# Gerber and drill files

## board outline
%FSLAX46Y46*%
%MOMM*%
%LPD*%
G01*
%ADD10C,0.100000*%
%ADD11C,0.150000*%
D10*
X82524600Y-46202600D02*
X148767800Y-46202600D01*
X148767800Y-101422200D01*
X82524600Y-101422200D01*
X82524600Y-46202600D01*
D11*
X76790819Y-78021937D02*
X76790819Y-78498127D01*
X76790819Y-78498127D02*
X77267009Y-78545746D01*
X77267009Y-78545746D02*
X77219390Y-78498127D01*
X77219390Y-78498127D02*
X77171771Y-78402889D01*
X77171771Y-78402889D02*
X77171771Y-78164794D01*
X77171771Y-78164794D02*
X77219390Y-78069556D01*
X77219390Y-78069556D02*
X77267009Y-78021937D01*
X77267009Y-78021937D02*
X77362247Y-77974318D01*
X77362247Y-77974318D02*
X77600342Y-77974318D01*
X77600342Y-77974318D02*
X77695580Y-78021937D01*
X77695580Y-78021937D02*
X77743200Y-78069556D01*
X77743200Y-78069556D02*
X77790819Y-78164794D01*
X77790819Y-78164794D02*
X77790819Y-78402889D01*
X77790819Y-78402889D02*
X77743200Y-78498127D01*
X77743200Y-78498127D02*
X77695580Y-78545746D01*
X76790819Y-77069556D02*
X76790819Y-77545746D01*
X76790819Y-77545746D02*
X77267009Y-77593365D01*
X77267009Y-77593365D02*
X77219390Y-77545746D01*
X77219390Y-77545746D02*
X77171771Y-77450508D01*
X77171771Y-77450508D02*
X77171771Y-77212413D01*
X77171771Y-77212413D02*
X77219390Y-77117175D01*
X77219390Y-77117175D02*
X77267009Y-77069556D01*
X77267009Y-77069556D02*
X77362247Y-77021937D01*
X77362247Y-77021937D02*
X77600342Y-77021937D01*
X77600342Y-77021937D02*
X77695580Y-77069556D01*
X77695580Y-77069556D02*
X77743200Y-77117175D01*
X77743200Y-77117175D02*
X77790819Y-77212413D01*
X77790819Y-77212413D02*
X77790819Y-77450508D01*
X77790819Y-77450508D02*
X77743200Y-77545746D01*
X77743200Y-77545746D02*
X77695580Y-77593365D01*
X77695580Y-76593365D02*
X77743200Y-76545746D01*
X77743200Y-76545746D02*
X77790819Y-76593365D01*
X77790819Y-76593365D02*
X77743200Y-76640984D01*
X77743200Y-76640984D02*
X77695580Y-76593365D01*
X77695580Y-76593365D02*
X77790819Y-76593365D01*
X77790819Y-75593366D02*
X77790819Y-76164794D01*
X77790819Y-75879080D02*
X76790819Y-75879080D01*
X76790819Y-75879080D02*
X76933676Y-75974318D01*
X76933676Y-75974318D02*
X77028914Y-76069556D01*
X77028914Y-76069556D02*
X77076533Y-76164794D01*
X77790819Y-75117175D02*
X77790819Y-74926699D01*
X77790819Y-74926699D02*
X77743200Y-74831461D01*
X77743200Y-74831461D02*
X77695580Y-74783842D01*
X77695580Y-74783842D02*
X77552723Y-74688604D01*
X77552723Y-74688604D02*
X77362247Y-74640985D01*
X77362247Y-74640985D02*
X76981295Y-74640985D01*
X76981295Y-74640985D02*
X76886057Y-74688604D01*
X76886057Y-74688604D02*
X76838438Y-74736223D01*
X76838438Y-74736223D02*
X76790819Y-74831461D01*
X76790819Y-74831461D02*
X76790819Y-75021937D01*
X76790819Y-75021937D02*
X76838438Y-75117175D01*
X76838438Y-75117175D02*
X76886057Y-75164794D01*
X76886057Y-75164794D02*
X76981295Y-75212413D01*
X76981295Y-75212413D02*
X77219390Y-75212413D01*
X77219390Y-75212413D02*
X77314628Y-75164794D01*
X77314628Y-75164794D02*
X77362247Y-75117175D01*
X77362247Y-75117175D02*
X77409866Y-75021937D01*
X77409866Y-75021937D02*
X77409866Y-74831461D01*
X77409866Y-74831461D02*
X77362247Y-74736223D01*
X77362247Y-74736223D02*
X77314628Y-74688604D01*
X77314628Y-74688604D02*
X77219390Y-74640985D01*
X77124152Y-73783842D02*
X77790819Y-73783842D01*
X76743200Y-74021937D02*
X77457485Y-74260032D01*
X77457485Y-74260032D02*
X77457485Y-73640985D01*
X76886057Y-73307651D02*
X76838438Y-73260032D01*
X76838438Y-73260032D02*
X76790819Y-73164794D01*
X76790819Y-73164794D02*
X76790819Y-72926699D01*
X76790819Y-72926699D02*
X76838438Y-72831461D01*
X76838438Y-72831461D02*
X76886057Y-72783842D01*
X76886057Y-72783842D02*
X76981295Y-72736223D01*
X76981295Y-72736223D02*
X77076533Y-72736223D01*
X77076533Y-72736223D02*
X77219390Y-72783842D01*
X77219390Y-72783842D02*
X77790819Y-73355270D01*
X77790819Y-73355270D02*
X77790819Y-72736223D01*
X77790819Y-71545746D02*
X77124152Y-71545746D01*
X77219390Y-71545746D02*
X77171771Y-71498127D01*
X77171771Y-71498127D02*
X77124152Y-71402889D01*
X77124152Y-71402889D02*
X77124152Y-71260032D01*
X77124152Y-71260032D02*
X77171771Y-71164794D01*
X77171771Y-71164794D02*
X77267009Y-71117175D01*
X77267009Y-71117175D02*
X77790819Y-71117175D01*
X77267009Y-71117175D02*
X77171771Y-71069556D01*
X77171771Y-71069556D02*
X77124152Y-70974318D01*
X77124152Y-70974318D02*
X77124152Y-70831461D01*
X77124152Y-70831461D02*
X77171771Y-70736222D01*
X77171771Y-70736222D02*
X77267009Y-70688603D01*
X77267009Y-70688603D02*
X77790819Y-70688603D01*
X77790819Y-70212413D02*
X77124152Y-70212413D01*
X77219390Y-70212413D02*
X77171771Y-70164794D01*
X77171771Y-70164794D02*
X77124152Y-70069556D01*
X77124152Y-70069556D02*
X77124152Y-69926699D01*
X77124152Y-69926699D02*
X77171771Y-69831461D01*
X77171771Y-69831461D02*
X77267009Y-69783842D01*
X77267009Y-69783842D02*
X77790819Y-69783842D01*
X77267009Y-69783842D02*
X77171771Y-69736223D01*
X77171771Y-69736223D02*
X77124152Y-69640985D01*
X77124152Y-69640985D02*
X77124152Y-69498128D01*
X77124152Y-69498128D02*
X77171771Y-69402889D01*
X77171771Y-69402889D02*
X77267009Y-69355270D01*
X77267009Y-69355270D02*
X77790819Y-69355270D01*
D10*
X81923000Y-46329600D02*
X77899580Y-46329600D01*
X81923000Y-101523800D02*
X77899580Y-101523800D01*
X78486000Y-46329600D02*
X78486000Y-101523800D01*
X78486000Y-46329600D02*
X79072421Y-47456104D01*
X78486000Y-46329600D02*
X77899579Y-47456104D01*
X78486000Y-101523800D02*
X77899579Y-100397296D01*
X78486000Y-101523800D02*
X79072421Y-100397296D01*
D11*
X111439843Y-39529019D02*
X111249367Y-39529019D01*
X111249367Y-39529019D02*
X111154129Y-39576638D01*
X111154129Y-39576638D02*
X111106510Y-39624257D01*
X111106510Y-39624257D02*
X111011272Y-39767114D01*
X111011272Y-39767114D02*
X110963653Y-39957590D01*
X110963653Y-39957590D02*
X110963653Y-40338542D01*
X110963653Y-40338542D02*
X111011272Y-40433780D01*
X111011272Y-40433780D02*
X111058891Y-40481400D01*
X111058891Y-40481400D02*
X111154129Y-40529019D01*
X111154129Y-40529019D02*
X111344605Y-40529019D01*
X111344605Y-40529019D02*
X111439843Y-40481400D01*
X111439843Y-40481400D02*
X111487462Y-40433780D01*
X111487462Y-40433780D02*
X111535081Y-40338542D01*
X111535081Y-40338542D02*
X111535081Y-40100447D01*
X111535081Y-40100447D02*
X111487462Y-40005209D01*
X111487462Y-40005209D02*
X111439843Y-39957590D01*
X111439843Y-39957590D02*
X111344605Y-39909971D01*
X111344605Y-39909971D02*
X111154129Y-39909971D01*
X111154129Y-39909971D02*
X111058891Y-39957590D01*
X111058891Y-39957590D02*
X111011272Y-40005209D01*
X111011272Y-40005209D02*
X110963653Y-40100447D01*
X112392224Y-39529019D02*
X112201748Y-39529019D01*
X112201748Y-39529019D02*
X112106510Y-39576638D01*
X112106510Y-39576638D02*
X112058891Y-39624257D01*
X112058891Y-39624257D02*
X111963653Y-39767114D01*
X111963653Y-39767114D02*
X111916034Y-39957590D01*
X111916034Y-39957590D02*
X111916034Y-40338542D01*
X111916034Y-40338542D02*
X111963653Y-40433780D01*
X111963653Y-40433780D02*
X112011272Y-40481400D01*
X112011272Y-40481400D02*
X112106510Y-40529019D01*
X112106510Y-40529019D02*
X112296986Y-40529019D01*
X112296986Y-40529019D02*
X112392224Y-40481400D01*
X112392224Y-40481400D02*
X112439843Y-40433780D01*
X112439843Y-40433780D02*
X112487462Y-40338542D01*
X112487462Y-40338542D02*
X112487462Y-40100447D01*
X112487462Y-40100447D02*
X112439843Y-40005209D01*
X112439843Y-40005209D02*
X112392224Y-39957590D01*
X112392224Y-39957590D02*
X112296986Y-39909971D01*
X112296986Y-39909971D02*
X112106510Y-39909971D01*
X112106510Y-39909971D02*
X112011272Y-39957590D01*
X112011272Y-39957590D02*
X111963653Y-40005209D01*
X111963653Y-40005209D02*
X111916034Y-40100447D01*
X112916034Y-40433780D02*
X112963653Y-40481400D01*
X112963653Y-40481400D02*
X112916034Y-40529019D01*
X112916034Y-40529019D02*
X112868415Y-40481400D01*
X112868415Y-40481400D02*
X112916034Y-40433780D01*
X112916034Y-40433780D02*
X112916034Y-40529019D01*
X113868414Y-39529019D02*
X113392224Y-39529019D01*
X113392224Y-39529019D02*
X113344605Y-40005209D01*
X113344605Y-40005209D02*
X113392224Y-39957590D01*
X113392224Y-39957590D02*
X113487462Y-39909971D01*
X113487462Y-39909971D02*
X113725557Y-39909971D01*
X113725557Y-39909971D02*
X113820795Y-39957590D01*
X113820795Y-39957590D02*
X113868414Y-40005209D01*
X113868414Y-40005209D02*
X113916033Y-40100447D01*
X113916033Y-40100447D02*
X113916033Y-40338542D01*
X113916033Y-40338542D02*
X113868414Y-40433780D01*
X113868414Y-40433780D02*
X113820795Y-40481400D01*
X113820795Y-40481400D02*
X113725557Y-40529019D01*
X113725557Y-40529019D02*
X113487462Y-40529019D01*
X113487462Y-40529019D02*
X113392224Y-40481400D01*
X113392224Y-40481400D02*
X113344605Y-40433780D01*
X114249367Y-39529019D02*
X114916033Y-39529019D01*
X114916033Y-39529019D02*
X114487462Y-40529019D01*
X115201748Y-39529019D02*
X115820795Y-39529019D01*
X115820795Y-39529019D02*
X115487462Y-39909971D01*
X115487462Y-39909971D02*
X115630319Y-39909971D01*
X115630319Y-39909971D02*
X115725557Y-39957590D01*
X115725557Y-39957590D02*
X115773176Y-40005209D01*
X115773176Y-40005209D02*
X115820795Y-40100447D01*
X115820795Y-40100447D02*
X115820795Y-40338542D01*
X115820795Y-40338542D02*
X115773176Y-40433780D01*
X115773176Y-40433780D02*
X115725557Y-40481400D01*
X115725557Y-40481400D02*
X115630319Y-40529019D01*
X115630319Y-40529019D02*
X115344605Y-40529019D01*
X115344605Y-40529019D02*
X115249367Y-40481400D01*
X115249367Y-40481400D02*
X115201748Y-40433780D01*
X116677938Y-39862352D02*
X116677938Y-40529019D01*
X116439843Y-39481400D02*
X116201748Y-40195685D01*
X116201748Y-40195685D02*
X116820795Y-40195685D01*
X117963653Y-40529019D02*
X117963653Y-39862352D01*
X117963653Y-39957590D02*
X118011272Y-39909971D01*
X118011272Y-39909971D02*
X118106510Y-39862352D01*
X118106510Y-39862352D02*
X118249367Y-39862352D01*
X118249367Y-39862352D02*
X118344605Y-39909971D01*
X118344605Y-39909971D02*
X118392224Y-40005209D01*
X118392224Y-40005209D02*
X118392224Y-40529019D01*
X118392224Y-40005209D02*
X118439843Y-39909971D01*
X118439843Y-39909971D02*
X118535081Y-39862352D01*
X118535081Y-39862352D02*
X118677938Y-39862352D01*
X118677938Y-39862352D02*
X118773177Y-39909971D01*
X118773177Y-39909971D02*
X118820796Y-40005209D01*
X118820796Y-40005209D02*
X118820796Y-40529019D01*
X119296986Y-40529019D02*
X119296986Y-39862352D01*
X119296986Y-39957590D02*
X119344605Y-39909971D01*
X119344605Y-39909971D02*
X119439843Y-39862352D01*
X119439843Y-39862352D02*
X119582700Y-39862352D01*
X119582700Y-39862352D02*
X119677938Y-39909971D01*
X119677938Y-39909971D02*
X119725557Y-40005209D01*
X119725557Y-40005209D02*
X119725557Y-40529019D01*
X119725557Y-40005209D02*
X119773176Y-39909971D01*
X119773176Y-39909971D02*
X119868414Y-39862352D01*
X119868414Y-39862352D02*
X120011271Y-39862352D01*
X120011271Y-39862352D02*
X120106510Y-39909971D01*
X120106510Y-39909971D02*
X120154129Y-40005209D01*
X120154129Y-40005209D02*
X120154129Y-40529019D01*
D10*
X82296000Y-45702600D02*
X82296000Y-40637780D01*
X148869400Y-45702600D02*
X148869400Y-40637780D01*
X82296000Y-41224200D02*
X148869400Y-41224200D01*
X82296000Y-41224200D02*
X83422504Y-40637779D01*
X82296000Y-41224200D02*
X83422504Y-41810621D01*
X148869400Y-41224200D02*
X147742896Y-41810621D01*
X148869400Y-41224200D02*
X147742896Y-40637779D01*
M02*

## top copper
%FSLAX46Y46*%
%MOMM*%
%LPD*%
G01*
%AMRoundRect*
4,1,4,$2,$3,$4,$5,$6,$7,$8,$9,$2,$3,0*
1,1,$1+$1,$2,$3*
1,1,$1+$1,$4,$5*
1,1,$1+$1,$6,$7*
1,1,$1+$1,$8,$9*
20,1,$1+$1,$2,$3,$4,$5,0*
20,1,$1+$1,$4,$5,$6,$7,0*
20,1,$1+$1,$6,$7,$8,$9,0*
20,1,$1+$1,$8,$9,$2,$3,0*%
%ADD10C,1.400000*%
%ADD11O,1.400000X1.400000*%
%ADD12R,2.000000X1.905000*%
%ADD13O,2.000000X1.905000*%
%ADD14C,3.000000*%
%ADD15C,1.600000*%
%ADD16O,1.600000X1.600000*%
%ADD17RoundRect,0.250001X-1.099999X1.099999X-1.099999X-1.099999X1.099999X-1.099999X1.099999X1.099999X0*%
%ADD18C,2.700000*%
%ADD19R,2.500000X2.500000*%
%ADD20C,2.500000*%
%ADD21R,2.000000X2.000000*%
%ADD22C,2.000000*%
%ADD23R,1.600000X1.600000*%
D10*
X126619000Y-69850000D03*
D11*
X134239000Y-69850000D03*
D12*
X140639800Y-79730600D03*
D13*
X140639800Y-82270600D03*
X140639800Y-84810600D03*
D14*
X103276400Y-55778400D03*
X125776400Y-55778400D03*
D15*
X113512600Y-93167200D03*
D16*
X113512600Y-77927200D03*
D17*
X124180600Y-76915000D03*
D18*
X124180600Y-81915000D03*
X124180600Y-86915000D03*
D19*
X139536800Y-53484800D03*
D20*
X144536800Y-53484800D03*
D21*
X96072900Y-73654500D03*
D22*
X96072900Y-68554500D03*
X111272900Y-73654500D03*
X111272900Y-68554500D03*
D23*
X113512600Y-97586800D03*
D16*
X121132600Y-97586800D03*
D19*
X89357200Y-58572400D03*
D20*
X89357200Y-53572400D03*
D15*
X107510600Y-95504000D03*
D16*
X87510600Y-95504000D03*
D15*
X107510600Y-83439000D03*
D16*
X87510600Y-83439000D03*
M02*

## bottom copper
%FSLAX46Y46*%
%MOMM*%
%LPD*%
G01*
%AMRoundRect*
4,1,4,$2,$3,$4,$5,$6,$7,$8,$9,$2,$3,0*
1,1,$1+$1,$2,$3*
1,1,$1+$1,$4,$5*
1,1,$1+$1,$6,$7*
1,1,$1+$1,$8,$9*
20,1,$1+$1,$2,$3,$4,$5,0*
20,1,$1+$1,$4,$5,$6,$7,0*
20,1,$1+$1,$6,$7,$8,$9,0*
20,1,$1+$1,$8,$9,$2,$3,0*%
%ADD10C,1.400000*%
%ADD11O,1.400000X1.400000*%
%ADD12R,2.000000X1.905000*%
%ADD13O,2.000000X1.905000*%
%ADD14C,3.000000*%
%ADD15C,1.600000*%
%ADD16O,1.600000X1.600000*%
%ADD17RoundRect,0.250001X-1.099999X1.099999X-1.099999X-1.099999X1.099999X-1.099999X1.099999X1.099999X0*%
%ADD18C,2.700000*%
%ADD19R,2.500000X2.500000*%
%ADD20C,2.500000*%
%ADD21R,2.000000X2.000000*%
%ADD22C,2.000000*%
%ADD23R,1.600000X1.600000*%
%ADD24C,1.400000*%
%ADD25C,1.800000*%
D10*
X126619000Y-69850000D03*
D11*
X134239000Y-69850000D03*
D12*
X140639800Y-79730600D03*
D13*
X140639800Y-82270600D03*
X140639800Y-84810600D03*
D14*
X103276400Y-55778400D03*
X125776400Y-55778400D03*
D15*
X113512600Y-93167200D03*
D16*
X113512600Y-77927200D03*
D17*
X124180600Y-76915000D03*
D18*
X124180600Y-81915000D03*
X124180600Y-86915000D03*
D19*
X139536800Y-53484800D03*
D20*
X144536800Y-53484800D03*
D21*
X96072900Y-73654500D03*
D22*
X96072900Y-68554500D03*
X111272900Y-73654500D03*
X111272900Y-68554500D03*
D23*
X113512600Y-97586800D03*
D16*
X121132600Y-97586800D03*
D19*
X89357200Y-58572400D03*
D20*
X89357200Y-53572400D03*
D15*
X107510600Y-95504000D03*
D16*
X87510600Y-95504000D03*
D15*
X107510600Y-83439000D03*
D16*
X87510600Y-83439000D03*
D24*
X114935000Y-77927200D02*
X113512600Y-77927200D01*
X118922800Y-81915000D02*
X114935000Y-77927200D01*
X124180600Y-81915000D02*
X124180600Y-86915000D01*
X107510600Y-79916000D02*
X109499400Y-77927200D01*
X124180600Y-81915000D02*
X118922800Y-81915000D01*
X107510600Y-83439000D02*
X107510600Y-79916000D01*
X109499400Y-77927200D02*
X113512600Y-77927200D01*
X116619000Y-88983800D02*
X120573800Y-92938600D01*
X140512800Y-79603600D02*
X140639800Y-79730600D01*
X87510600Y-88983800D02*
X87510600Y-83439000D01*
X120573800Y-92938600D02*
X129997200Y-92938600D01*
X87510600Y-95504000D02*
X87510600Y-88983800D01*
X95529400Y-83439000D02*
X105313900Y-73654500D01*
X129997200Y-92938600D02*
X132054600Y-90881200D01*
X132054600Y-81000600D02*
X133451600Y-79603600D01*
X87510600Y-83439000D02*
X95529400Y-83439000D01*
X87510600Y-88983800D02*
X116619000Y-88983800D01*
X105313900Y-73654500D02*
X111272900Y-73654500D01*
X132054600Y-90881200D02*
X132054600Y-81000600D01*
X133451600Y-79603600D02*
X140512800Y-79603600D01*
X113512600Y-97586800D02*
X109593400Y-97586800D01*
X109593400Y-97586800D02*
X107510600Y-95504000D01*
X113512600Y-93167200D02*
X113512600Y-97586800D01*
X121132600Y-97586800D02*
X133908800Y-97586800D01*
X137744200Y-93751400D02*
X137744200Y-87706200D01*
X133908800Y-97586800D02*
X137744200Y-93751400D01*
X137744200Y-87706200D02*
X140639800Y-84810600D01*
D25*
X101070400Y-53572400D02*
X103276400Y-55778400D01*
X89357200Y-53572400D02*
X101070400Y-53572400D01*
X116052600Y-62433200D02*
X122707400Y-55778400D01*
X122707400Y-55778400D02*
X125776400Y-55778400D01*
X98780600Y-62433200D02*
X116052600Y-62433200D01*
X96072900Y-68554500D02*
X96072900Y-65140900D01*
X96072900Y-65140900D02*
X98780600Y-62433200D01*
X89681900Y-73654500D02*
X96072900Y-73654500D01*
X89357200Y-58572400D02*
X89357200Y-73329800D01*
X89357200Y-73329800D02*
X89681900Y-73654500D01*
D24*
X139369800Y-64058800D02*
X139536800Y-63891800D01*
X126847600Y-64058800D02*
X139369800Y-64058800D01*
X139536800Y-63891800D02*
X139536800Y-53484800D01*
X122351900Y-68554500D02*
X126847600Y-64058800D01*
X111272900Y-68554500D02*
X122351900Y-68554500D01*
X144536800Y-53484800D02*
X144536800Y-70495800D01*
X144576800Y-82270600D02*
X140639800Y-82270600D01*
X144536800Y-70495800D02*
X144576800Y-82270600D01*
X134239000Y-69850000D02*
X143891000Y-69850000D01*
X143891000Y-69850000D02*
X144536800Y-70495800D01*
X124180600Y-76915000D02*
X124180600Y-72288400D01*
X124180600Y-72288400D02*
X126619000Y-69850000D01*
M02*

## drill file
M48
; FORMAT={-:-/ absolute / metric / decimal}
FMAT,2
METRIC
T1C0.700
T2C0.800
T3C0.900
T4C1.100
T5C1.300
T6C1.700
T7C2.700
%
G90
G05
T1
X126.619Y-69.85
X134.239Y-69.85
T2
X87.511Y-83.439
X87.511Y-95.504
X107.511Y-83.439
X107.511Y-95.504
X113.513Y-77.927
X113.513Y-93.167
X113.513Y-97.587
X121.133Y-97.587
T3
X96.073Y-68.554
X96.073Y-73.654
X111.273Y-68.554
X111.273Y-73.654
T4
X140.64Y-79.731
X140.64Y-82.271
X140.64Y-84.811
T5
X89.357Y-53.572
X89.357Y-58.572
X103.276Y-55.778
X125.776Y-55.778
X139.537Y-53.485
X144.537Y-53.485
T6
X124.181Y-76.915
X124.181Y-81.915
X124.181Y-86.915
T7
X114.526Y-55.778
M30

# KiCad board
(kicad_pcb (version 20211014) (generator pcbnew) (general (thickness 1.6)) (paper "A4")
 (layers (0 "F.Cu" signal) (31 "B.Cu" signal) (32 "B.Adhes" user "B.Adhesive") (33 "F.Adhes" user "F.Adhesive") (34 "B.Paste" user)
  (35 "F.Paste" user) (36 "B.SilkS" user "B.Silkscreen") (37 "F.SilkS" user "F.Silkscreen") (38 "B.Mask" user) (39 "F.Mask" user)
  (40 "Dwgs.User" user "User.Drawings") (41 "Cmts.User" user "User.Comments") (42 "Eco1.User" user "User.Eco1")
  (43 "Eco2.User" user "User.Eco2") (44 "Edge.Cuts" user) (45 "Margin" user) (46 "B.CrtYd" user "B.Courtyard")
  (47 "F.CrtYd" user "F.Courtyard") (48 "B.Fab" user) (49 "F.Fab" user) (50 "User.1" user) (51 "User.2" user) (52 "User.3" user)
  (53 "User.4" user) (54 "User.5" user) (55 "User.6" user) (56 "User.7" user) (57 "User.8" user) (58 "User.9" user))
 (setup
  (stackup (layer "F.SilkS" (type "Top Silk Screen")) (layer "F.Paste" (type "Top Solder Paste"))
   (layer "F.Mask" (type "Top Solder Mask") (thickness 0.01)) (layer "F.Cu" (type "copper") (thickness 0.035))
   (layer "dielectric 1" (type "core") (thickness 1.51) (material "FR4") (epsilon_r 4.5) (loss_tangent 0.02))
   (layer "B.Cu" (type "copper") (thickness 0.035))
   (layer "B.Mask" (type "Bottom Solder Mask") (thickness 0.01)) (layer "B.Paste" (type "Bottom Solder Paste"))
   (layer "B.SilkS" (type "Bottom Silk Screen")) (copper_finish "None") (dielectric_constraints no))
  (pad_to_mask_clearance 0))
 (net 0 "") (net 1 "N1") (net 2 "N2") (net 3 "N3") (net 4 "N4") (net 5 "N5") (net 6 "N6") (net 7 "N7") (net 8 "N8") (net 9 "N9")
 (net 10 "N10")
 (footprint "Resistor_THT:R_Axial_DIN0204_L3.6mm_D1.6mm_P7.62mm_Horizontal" (layer "F.Cu") (at 126.619 69.85)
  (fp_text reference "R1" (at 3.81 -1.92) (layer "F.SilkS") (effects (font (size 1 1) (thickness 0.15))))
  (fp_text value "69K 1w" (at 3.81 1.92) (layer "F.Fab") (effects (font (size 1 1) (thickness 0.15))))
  (pad "1" thru_hole circle (at 0 0) (size 1.4 1.4) (drill 0.7) (layers *.Cu *.Mask) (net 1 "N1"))
  (pad "2" thru_hole oval (at 7.62 0) (size 1.4 1.4) (drill 0.7) (layers *.Cu *.Mask) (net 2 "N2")))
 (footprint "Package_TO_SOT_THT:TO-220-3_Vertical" (layer "F.Cu") (at 140.6398 79.7306 -90)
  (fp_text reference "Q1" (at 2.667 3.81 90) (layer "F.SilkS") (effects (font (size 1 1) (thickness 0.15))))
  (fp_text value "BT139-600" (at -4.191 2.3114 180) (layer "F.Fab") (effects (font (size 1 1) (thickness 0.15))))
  (pad "1" thru_hole rect (at 0 0 270) (size 1.905 2) (drill 1.1) (layers *.Cu *.Mask) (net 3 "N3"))
  (pad "2" thru_hole oval (at 2.54 0 270) (size 1.905 2) (drill 1.1) (layers *.Cu *.Mask) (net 2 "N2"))
  (pad "3" thru_hole oval (at 5.08 0 270) (size 1.905 2) (drill 1.1) (layers *.Cu *.Mask) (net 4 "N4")))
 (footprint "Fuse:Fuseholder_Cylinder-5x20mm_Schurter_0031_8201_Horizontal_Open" (layer "F.Cu") (at 103.2764 55.7784)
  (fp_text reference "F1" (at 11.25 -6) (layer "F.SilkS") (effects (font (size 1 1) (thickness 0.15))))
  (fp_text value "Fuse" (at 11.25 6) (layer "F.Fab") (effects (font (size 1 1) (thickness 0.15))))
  (pad "" np_thru_hole circle (at 11.25 0) (size 2.7 2.7) (drill 2.7) (layers *.Cu *.Mask))
  (pad "1" thru_hole circle (at 0 0) (size 3 3) (drill 1.3) (layers *.Cu *.Mask) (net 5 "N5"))
  (pad "2" thru_hole circle (at 22.5 0) (size 3 3) (drill 1.3) (layers *.Cu *.Mask) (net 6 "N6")))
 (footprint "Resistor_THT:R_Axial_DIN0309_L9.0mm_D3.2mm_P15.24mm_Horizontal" (layer "F.Cu") (at 113.5126 93.1672 90)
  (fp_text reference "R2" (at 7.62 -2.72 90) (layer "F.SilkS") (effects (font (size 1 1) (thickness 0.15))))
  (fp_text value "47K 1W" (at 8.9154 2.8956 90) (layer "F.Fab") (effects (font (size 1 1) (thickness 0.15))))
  (pad "1" thru_hole circle (at 0 0 90) (size 1.6 1.6) (drill 0.8) (layers *.Cu *.Mask) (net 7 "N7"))
  (pad "2" thru_hole oval (at 15.24 0 90) (size 1.6 1.6) (drill 0.8) (layers *.Cu *.Mask) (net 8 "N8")))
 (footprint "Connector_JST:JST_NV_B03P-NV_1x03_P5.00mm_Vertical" (layer "F.Cu") (at 124.1806 76.915 -90)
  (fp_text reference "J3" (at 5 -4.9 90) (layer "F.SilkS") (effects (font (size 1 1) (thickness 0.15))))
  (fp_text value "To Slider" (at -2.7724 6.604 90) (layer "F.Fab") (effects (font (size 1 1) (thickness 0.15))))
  (pad "1" thru_hole roundrect (at 0 0 270) (size 2.7 2.7) (drill 1.7) (layers *.Cu *.Mask) (roundrect_rratio 0.092593) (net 1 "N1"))
  (pad "2" thru_hole circle (at 5 0 270) (size 2.7 2.7) (drill 1.7) (layers *.Cu *.Mask) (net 8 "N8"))
  (pad "3" thru_hole circle (at 10 0 270) (size 2.7 2.7) (drill 1.7) (layers *.Cu *.Mask) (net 8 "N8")))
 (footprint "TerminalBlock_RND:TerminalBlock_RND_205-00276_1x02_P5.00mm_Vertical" (layer "F.Cu") (at 139.5368 53.4848)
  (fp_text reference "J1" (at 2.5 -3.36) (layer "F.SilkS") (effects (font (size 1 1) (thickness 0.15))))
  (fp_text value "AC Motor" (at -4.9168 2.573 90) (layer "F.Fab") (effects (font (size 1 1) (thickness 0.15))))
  (pad "1" thru_hole rect (at 0 0) (size 2.5 2.5) (drill 1.3) (layers *.Cu *.Mask) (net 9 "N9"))
  (pad "2" thru_hole circle (at 5 0) (size 2.5 2.5) (drill 1.3) (layers *.Cu *.Mask) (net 2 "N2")))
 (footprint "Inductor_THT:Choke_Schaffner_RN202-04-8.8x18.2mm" (layer "F.Cu") (at 96.0729 73.6545 90)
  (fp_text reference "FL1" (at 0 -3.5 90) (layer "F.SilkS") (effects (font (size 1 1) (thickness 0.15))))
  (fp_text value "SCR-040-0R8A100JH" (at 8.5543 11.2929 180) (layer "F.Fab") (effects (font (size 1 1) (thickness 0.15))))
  (pad "1" thru_hole rect (at 0 0 90) (size 2 2) (drill 0.9) (layers *.Cu *.Mask) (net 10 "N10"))
  (pad "2" thru_hole circle (at 5.1 0 90) (size 2 2) (drill 0.9) (layers *.Cu *.Mask) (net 6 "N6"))
  (pad "3" thru_hole circle (at 0 15.2 90) (size 2 2) (drill 0.9) (layers *.Cu *.Mask) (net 3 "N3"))
  (pad "4" thru_hole circle (at 5.1 15.2 90) (size 2 2) (drill 0.9) (layers *.Cu *.Mask) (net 9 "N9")))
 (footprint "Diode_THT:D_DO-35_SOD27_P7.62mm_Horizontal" (layer "F.Cu") (at 113.5126 97.5868)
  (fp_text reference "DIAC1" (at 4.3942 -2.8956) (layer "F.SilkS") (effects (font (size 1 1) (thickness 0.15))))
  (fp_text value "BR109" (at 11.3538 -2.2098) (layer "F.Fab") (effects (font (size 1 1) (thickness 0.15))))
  (pad "1" thru_hole rect (at 0 0) (size 1.6 1.6) (drill 0.8) (layers *.Cu *.Mask) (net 7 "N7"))
  (pad "2" thru_hole oval (at 7.62 0) (size 1.6 1.6) (drill 0.8) (layers *.Cu *.Mask) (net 4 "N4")))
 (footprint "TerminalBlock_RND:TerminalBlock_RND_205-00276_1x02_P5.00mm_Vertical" (layer "F.Cu") (at 89.3572 58.5724 90)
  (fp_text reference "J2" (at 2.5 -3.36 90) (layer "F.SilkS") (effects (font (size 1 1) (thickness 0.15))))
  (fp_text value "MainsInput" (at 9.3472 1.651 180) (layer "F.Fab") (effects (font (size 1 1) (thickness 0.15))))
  (pad "1" thru_hole rect (at 0 0 90) (size 2.5 2.5) (drill 1.3) (layers *.Cu *.Mask) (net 10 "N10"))
  (pad "2" thru_hole circle (at 5 0 90) (size 2.5 2.5) (drill 1.3) (layers *.Cu *.Mask) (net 5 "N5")))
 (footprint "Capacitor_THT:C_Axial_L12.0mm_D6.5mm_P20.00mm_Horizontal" (layer "F.Cu") (at 107.5106 95.504 180)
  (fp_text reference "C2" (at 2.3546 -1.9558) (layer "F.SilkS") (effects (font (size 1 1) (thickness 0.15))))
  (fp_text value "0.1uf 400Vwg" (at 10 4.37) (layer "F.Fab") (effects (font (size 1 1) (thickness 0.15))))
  (pad "1" thru_hole circle (at 0 0 180) (size 1.6 1.6) (drill 0.8) (layers *.Cu *.Mask) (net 7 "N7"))
  (pad "2" thru_hole oval (at 20 0 180) (size 1.6 1.6) (drill 0.8) (layers *.Cu *.Mask) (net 3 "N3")))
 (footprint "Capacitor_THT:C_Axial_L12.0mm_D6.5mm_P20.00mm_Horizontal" (layer "F.Cu") (at 107.5106 83.439 180)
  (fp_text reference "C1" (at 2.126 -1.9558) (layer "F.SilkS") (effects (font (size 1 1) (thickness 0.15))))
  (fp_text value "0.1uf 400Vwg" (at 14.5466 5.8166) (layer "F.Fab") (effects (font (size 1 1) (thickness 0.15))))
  (pad "1" thru_hole circle (at 0 0 180) (size 1.6 1.6) (drill 0.8) (layers *.Cu *.Mask) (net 8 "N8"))
  (pad "2" thru_hole oval (at 20 0 180) (size 1.6 1.6) (drill 0.8) (layers *.Cu *.Mask) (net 3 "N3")))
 (gr_rect (start 82.5246 46.2026) (end 148.7678 101.4222) (layer "Edge.Cuts") (width 0.1) (fill none))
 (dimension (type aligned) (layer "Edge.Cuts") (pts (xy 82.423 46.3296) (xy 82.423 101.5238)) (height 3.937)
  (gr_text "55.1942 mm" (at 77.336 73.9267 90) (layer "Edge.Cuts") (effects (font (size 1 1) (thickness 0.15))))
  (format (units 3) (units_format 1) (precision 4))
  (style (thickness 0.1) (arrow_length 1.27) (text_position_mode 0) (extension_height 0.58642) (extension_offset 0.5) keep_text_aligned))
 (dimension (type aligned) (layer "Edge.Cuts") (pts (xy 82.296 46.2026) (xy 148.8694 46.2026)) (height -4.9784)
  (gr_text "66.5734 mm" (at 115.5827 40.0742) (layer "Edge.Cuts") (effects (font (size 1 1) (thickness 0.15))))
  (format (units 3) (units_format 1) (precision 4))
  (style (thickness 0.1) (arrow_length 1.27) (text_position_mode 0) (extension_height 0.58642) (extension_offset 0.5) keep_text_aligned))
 (segment (start 114.935 77.9272) (end 113.5126 77.9272) (width 1.4) (layer "B.Cu") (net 8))
 (segment (start 118.9228 81.915) (end 114.935 77.9272) (width 1.4) (layer "B.Cu") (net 8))
 (segment (start 124.1806 81.915) (end 124.1806 86.915) (width 1.4) (layer "B.Cu") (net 8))
 (segment (start 107.5106 79.916) (end 109.4994 77.9272) (width 1.4) (layer "B.Cu") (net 8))
 (segment (start 124.1806 81.915) (end 118.9228 81.915) (width 1.4) (layer "B.Cu") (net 8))
 (segment (start 107.5106 83.439) (end 107.5106 79.916) (width 1.4) (layer "B.Cu") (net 8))
 (segment (start 109.4994 77.9272) (end 113.5126 77.9272) (width 1.4) (layer "B.Cu") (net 8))
 (segment (start 116.619 88.9838) (end 120.5738 92.9386) (width 1.4) (layer "B.Cu") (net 3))
 (segment (start 140.5128 79.6036) (end 140.6398 79.7306) (width 1.4) (layer "B.Cu") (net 3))
 (segment (start 87.5106 88.9838) (end 87.5106 83.439) (width 1.4) (layer "B.Cu") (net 3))
 (segment (start 120.5738 92.9386) (end 129.9972 92.9386) (width 1.4) (layer "B.Cu") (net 3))
 (segment (start 87.5106 95.504) (end 87.5106 88.9838) (width 1.4) (layer "B.Cu") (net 3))
 (segment (start 95.5294 83.439) (end 105.3139 73.6545) (width 1.4) (layer "B.Cu") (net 3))
 (segment (start 129.9972 92.9386) (end 132.0546 90.8812) (width 1.4) (layer "B.Cu") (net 3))
 (segment (start 132.0546 81.0006) (end 133.4516 79.6036) (width 1.4) (layer "B.Cu") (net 3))
 (segment (start 87.5106 83.439) (end 95.5294 83.439) (width 1.4) (layer "B.Cu") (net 3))
 (segment (start 87.5106 88.9838) (end 116.619 88.9838) (width 1.4) (layer "B.Cu") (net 3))
 (segment (start 105.3139 73.6545) (end 111.2729 73.6545) (width 1.4) (layer "B.Cu") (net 3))
 (segment (start 132.0546 90.8812) (end 132.0546 81.0006) (width 1.4) (layer "B.Cu") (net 3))
 (segment (start 133.4516 79.6036) (end 140.5128 79.6036) (width 1.4) (layer "B.Cu") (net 3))
 (segment (start 113.5126 97.5868) (end 109.5934 97.5868) (width 1.4) (layer "B.Cu") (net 7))
 (segment (start 109.5934 97.5868) (end 107.5106 95.504) (width 1.4) (layer "B.Cu") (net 7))
 (segment (start 113.5126 93.1672) (end 113.5126 97.5868) (width 1.4) (layer "B.Cu") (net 7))
 (segment (start 121.1326 97.5868) (end 133.9088 97.5868) (width 1.4) (layer "B.Cu") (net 4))
 (segment (start 137.7442 93.7514) (end 137.7442 87.7062) (width 1.4) (layer "B.Cu") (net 4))
 (segment (start 133.9088 97.5868) (end 137.7442 93.7514) (width 1.4) (layer "B.Cu") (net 4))
 (segment (start 137.7442 87.7062) (end 140.6398 84.8106) (width 1.4) (layer "B.Cu") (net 4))
 (segment (start 101.0704 53.5724) (end 103.2764 55.7784) (width 1.8) (layer "B.Cu") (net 5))
 (segment (start 89.3572 53.5724) (end 101.0704 53.5724) (width 1.8) (layer "B.Cu") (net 5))
 (segment (start 116.0526 62.4332) (end 122.7074 55.7784) (width 1.8) (layer "B.Cu") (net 6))
 (segment (start 122.7074 55.7784) (end 125.7764 55.7784) (width 1.8) (layer "B.Cu") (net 6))
 (segment (start 98.7806 62.4332) (end 116.0526 62.4332) (width 1.8) (layer "B.Cu") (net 6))
 (segment (start 96.0729 68.5545) (end 96.0729 65.1409) (width 1.8) (layer "B.Cu") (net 6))
 (segment (start 96.0729 65.1409) (end 98.7806 62.4332) (width 1.8) (layer "B.Cu") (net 6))
 (segment (start 89.6819 73.6545) (end 96.0729 73.6545) (width 1.8) (layer "B.Cu") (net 10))
 (segment (start 89.3572 58.5724) (end 89.3572 73.3298) (width 1.8) (layer "B.Cu") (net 10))
 (segment (start 89.3572 73.3298) (end 89.6819 73.6545) (width 1.8) (layer "B.Cu") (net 10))
 (segment (start 139.3698 64.0588) (end 139.5368 63.8918) (width 1.4) (layer "B.Cu") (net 9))
 (segment (start 126.8476 64.0588) (end 139.3698 64.0588) (width 1.4) (layer "B.Cu") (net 9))
 (segment (start 139.5368 63.8918) (end 139.5368 53.4848) (width 1.4) (layer "B.Cu") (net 9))
 (segment (start 122.3519 68.5545) (end 126.8476 64.0588) (width 1.4) (layer "B.Cu") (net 9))
 (segment (start 111.2729 68.5545) (end 122.3519 68.5545) (width 1.4) (layer "B.Cu") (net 9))
 (segment (start 144.5368 53.4848) (end 144.5368 70.4958) (width 1.4) (layer "B.Cu") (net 2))
 (segment (start 144.5768 82.2706) (end 140.6398 82.2706) (width 1.4) (layer "B.Cu") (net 2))
 (segment (start 144.5368 70.4958) (end 144.5768 82.2706) (width 1.4) (layer "B.Cu") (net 2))
 (segment (start 134.239 69.85) (end 143.891 69.85) (width 1.4) (layer "B.Cu") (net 2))
 (segment (start 143.891 69.85) (end 144.5368 70.4958) (width 1.4) (layer "B.Cu") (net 2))
 (segment (start 124.1806 76.915) (end 124.1806 72.2884) (width 1.4) (layer "B.Cu") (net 1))
 (segment (start 124.1806 72.2884) (end 126.619 69.85) (width 1.4) (layer "B.Cu") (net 1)))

